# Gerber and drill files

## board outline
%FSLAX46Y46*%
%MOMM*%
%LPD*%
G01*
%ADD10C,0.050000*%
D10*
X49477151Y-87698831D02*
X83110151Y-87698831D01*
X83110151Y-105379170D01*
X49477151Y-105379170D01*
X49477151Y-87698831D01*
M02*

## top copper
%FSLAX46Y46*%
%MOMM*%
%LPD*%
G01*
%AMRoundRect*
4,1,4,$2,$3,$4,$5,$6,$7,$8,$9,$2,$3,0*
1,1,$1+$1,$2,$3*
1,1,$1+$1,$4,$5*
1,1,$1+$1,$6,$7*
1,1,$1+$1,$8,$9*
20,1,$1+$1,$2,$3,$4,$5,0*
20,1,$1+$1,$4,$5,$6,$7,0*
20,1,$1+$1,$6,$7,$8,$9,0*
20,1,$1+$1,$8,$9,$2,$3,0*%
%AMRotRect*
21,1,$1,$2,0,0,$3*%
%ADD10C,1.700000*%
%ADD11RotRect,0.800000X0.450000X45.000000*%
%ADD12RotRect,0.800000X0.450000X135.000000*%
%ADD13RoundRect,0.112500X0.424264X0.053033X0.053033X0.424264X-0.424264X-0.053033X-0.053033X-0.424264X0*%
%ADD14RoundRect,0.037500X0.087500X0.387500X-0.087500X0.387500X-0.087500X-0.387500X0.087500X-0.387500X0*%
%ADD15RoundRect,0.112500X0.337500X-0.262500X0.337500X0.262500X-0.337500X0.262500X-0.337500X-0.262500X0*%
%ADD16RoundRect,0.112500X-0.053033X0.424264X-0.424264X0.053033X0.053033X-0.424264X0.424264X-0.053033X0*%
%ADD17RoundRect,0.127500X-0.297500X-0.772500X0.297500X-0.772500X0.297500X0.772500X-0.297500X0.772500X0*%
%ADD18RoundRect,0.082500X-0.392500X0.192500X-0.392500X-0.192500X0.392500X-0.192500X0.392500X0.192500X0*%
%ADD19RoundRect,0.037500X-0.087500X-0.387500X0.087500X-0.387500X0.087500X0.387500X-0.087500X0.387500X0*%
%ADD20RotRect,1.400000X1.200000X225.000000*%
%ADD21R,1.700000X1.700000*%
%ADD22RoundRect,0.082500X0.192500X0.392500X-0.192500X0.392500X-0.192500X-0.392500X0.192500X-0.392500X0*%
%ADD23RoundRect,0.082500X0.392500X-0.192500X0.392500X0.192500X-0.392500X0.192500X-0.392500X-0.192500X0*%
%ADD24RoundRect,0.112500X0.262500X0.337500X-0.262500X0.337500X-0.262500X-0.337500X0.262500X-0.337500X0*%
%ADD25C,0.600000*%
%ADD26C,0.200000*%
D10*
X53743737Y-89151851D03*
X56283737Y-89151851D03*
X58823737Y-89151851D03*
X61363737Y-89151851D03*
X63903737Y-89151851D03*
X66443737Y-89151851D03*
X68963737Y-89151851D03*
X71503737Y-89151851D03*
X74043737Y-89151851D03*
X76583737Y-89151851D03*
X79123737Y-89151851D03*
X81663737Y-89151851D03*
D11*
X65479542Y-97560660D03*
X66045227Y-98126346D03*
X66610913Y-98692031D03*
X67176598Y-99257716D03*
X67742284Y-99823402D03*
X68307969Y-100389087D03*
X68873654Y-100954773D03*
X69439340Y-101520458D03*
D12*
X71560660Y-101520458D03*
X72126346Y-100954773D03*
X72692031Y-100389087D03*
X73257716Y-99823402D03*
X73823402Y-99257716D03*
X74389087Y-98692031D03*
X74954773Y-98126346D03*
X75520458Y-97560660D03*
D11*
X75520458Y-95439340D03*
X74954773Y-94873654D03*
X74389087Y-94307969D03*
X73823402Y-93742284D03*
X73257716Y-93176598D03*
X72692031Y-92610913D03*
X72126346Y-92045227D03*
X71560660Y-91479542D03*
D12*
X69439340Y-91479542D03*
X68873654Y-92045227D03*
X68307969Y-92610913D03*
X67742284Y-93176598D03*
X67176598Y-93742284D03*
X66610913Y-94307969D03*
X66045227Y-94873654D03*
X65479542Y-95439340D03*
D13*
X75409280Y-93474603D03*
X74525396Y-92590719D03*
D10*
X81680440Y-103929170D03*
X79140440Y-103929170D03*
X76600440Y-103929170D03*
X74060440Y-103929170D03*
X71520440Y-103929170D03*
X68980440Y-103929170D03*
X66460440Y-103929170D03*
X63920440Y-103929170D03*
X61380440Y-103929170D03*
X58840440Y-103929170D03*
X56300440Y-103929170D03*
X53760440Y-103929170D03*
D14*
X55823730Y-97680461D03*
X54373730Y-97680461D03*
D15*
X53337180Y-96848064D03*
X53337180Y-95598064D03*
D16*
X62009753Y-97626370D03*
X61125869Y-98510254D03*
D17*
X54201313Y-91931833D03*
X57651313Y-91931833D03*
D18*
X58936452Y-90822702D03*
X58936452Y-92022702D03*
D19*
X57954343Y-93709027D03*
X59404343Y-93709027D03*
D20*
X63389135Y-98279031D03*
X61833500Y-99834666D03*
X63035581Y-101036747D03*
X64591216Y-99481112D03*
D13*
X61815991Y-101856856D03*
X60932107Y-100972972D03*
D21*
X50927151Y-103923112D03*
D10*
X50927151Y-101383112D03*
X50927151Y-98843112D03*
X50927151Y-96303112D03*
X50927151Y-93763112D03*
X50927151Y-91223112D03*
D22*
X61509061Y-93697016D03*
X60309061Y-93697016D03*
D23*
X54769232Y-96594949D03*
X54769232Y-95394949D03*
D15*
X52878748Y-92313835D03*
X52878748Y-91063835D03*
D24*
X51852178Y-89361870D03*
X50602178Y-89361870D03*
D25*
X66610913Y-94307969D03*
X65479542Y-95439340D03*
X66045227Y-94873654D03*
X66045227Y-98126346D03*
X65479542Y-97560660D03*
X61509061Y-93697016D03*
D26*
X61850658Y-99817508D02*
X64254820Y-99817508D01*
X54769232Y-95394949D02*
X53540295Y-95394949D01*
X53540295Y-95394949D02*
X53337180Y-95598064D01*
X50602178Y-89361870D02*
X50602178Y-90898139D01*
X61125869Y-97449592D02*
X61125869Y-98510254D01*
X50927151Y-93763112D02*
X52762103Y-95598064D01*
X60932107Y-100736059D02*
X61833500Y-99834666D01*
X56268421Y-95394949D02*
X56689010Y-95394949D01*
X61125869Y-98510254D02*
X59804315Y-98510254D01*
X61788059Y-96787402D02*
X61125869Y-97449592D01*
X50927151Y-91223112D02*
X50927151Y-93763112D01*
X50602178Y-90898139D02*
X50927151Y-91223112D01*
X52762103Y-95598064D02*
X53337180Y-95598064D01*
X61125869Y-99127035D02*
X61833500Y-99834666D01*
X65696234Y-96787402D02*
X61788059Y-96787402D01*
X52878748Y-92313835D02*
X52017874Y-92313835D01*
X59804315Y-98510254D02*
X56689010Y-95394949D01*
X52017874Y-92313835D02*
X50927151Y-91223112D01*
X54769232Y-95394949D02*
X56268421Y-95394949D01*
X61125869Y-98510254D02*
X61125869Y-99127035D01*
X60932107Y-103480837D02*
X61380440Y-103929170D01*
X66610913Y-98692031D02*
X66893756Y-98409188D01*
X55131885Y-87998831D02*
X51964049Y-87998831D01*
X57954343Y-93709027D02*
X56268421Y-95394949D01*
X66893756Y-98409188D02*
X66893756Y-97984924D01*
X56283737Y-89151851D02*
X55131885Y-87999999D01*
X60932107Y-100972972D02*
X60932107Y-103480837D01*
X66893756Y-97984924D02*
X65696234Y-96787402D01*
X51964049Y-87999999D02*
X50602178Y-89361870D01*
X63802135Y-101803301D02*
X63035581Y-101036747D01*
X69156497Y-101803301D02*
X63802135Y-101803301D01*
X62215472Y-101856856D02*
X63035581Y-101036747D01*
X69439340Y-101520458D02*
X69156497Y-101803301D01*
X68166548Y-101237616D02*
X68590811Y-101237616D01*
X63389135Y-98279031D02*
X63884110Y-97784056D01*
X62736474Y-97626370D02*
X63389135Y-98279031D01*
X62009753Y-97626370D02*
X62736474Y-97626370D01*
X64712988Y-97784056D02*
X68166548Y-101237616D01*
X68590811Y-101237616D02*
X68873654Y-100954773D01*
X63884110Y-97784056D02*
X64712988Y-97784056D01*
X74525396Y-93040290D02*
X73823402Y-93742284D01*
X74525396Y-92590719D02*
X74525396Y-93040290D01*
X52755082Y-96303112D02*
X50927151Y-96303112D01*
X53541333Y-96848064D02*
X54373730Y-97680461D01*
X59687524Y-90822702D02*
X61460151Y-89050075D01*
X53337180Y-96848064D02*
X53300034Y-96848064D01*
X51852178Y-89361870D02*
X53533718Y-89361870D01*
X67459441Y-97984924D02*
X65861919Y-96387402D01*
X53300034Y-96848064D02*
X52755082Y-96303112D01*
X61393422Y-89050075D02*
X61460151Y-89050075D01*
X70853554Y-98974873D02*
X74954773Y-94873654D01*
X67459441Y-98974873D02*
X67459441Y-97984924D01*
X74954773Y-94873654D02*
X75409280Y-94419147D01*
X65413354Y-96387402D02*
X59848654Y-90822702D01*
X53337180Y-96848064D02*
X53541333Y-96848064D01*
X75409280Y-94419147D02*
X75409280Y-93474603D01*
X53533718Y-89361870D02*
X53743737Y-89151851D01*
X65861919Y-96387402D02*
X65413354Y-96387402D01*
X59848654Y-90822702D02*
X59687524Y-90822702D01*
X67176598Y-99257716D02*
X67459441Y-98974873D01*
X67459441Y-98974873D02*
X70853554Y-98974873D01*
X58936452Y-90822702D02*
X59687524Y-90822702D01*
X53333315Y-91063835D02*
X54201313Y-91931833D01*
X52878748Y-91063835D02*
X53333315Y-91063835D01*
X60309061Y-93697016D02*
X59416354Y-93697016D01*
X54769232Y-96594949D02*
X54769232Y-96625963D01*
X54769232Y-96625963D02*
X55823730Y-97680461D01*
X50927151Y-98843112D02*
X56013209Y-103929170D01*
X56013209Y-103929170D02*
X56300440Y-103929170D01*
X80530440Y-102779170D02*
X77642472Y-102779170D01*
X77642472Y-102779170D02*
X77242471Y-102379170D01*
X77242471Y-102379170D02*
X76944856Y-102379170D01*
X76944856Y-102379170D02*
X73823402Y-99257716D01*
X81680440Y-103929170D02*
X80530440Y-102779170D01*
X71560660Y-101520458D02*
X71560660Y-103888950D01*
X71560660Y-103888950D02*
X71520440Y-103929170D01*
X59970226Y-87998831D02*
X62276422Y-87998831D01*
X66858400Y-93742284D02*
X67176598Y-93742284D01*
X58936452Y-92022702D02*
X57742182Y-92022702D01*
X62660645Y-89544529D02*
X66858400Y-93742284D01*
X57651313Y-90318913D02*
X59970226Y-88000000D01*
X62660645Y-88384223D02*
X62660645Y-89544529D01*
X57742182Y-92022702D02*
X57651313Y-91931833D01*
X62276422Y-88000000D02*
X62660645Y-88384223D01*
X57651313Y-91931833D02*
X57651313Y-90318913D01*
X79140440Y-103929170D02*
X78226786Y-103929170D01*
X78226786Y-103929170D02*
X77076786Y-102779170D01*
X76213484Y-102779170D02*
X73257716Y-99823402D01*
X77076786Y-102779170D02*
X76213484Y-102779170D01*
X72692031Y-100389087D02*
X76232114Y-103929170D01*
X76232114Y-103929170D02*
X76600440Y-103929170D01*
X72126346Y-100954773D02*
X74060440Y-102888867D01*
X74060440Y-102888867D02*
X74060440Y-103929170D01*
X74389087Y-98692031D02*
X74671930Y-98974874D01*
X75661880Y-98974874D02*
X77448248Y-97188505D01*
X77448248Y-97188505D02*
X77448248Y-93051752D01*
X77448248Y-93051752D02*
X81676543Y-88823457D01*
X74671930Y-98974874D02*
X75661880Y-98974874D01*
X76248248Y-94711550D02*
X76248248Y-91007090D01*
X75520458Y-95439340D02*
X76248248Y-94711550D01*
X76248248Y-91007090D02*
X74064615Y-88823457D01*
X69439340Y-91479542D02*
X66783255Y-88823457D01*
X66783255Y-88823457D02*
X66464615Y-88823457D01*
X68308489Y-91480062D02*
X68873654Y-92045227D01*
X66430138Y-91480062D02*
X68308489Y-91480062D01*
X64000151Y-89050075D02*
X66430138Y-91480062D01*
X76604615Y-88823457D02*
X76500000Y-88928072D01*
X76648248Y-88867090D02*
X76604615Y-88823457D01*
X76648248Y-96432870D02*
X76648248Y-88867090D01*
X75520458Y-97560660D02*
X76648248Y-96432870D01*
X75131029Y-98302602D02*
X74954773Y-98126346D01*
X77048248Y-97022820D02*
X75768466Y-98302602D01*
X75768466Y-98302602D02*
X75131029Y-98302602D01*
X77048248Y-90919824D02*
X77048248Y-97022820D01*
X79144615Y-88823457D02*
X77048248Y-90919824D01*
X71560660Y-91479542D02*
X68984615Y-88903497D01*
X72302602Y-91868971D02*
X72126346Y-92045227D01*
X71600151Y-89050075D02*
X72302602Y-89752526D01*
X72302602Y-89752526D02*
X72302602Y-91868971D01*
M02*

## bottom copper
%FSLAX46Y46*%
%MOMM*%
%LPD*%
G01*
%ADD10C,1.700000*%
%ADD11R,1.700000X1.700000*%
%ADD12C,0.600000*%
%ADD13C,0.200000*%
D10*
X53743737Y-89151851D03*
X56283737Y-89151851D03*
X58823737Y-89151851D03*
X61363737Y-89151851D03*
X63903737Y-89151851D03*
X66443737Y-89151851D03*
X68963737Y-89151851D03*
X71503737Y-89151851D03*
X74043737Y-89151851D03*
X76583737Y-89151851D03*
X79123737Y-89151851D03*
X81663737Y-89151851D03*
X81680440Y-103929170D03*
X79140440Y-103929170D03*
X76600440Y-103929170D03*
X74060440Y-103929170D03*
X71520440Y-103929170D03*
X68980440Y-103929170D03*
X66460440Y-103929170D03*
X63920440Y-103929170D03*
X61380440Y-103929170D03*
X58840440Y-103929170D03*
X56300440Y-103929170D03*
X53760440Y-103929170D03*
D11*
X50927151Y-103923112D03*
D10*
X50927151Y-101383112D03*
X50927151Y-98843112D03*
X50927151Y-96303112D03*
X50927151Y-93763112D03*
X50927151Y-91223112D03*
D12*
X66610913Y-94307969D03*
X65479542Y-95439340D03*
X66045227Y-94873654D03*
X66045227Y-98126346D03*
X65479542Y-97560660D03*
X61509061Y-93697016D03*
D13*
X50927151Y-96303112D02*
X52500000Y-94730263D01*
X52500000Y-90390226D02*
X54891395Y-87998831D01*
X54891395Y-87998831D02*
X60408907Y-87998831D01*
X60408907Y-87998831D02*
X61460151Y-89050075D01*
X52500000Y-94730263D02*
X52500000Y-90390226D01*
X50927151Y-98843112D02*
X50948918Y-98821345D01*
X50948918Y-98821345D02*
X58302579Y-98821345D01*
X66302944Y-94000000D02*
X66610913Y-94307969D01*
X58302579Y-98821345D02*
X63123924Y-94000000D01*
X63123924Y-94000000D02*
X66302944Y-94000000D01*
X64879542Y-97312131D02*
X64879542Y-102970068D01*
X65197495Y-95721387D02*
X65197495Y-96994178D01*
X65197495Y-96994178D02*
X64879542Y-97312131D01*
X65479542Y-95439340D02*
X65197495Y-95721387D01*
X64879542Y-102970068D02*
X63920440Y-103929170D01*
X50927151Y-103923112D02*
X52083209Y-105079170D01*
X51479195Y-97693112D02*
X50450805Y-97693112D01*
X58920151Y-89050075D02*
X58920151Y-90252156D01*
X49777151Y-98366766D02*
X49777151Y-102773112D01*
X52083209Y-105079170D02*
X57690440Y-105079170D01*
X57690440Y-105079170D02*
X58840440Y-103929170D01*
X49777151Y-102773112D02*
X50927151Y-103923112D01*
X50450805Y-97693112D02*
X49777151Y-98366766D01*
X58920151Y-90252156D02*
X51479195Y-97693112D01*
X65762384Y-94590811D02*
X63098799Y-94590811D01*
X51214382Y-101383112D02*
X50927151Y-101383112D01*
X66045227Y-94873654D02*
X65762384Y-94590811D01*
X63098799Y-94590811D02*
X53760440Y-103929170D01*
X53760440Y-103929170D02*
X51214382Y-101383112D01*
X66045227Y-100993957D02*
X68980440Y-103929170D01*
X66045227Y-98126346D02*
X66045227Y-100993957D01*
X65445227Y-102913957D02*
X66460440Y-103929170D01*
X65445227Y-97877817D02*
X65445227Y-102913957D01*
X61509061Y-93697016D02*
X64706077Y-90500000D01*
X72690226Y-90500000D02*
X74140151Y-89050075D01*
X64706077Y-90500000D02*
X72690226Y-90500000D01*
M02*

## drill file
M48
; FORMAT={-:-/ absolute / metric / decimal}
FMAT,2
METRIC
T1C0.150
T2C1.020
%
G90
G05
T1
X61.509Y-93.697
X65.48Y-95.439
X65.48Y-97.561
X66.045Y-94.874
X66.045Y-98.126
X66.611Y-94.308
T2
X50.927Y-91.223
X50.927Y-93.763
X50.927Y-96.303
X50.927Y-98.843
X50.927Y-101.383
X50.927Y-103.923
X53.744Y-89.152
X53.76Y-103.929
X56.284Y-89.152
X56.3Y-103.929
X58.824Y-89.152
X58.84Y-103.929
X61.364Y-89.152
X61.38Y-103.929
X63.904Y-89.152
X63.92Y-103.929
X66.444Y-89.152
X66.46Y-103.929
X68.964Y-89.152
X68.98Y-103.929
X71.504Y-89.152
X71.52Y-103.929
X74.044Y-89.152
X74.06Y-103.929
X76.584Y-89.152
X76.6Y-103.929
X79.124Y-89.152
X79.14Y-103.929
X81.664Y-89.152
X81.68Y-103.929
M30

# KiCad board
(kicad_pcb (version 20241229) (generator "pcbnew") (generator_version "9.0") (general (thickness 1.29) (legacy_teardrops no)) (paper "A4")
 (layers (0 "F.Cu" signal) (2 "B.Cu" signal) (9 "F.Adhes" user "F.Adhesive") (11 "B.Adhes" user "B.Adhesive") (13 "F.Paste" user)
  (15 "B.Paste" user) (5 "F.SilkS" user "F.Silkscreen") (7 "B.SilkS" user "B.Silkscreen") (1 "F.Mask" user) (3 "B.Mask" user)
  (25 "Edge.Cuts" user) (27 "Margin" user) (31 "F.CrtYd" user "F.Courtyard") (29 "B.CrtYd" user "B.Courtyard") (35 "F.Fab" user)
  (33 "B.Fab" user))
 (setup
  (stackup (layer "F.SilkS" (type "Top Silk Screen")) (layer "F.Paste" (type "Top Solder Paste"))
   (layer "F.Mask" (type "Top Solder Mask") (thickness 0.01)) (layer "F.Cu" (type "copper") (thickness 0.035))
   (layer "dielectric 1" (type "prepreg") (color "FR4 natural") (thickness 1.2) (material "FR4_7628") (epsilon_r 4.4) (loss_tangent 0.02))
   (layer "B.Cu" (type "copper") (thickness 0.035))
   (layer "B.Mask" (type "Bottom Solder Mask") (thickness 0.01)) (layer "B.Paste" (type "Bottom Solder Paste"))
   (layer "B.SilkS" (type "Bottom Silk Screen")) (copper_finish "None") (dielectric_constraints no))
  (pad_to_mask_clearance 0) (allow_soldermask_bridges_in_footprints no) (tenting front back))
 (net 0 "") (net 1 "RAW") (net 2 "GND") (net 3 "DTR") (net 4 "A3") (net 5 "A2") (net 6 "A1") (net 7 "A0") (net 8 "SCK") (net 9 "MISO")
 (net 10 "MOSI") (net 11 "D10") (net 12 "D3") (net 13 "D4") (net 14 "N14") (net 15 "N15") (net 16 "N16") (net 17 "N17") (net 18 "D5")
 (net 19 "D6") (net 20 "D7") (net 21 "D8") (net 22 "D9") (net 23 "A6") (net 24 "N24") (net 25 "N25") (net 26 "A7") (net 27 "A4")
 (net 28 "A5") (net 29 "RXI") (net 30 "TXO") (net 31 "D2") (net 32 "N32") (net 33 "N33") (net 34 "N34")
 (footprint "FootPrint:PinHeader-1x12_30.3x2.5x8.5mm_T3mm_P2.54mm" (layer "F.Cu") (at 67.703737 89.151851)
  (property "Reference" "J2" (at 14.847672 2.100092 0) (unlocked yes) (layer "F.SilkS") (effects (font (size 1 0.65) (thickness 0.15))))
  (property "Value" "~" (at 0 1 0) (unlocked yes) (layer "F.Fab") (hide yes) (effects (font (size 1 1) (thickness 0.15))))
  (pad "1" thru_hole circle (at -13.96 0) (size 1.7 1.7) (drill 1.02) (layers "*.Cu" "*.Mask") (remove_unused_layers no) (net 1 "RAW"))
  (pad "2" thru_hole circle (at -11.42 0) (size 1.7 1.7) (drill 1.02) (layers "*.Cu" "*.Mask") (remove_unused_layers no) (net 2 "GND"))
  (pad "3" thru_hole circle (at -8.88 0) (size 1.7 1.7) (drill 1.02) (layers "*.Cu" "*.Mask") (remove_unused_layers no) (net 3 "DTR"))
  (pad "4" thru_hole circle (at -6.34 0) (size 1.7 1.7) (drill 1.02) (layers "*.Cu" "*.Mask") (remove_unused_layers no) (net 1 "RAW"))
  (pad "5" thru_hole circle (at -3.8 0) (size 1.7 1.7) (drill 1.02) (layers "*.Cu" "*.Mask") (remove_unused_layers no) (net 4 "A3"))
  (pad "6" thru_hole circle (at -1.26 0) (size 1.7 1.7) (drill 1.02) (layers "*.Cu" "*.Mask") (remove_unused_layers no) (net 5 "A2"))
  (pad "7" thru_hole circle (at 1.26 0) (size 1.7 1.7) (drill 1.02) (layers "*.Cu" "*.Mask") (remove_unused_layers no) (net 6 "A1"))
  (pad "8" thru_hole circle (at 3.8 0) (size 1.7 1.7) (drill 1.02) (layers "*.Cu" "*.Mask") (remove_unused_layers no) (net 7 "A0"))
  (pad "9" thru_hole circle (at 6.34 0) (size 1.7 1.7) (drill 1.02) (layers "*.Cu" "*.Mask") (remove_unused_layers no) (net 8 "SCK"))
  (pad "10" thru_hole circle (at 8.88 0) (size 1.7 1.7) (drill 1.02) (layers "*.Cu" "*.Mask") (remove_unused_layers no) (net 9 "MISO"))
  (pad "11" thru_hole circle (at 11.42 0) (size 1.7 1.7) (drill 1.02) (layers "*.Cu" "*.Mask") (remove_unused_layers no) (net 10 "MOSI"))
  (pad "12" thru_hole circle (at 13.96 0) (size 1.7 1.7) (drill 1.02) (layers "*.Cu" "*.Mask") (remove_unused_layers no) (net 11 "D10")))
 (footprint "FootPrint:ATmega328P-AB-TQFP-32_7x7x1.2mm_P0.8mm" (layer "F.Cu") (at 70.5 96.5 45)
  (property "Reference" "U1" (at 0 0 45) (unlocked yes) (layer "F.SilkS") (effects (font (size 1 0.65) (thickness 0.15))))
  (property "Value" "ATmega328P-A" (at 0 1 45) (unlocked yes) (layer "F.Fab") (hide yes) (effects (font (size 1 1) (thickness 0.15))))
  (pad "1" smd rect (at -4.3 -2.8 45) (size 0.8 0.45) (layers "F.Cu" "F.Mask" "F.Paste") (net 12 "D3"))
  (pad "2" smd rect (at -4.3 -2 45) (size 0.8 0.45) (layers "F.Cu" "F.Mask" "F.Paste") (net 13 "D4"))
  (pad "3" smd rect (at -4.3 -1.2 45) (size 0.8 0.45) (layers "F.Cu" "F.Mask" "F.Paste") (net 2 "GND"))
  (pad "4" smd rect (at -4.3 -0.4 45) (size 0.8 0.45) (layers "F.Cu" "F.Mask" "F.Paste") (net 1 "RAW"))
  (pad "5" smd rect (at -4.3 0.4 45) (size 0.8 0.45) (layers "F.Cu" "F.Mask" "F.Paste") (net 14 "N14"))
  (pad "6" smd rect (at -4.3 1.2 45) (size 0.8 0.45) (layers "F.Cu" "F.Mask" "F.Paste") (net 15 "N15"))
  (pad "7" smd rect (at -4.3 2 45) (size 0.8 0.45) (layers "F.Cu" "F.Mask" "F.Paste") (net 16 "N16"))
  (pad "8" smd rect (at -4.3 2.8 45) (size 0.8 0.45) (layers "F.Cu" "F.Mask" "F.Paste") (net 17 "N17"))
  (pad "9" smd rect (at -2.8 4.3 135) (size 0.8 0.45) (layers "F.Cu" "F.Mask" "F.Paste") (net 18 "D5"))
  (pad "10" smd rect (at -2 4.3 135) (size 0.8 0.45) (layers "F.Cu" "F.Mask" "F.Paste") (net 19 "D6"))
  (pad "11" smd rect (at -1.2 4.3 135) (size 0.8 0.45) (layers "F.Cu" "F.Mask" "F.Paste") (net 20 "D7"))
  (pad "12" smd rect (at -0.4 4.3 135) (size 0.8 0.45) (layers "F.Cu" "F.Mask" "F.Paste") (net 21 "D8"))
  (pad "13" smd rect (at 0.4 4.3 135) (size 0.8 0.45) (layers "F.Cu" "F.Mask" "F.Paste") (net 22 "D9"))
  (pad "14" smd rect (at 1.2 4.3 135) (size 0.8 0.45) (layers "F.Cu" "F.Mask" "F.Paste") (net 11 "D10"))
  (pad "15" smd rect (at 2 4.3 135) (size 0.8 0.45) (layers "F.Cu" "F.Mask" "F.Paste") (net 10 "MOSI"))
  (pad "16" smd rect (at 2.8 4.3 135) (size 0.8 0.45) (layers "F.Cu" "F.Mask" "F.Paste") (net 9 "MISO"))
  (pad "17" smd rect (at 4.3 2.8 45) (size 0.8 0.45) (layers "F.Cu" "F.Mask" "F.Paste") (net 8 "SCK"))
  (pad "18" smd rect (at 4.3 2 45) (size 0.8 0.45) (layers "F.Cu" "F.Mask" "F.Paste") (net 1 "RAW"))
  (pad "19" smd rect (at 4.3 1.2 45) (size 0.8 0.45) (layers "F.Cu" "F.Mask" "F.Paste") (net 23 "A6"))
  (pad "20" smd rect (at 4.3 0.4 45) (size 0.8 0.45) (layers "F.Cu" "F.Mask" "F.Paste") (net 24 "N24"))
  (pad "21" smd rect (at 4.3 -0.4 45) (size 0.8 0.45) (layers "F.Cu" "F.Mask" "F.Paste") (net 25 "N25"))
  (pad "22" smd rect (at 4.3 -1.2 45) (size 0.8 0.45) (layers "F.Cu" "F.Mask" "F.Paste") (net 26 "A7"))
  (pad "23" smd rect (at 4.3 -2 45) (size 0.8 0.45) (layers "F.Cu" "F.Mask" "F.Paste") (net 7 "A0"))
  (pad "24" smd rect (at 4.3 -2.8 45) (size 0.8 0.45) (layers "F.Cu" "F.Mask" "F.Paste") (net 6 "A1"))
  (pad "25" smd rect (at 2.8 -4.3 135) (size 0.8 0.45) (layers "F.Cu" "F.Mask" "F.Paste") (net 5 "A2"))
  (pad "26" smd rect (at 2 -4.3 135) (size 0.8 0.45) (layers "F.Cu" "F.Mask" "F.Paste") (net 4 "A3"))
  (pad "27" smd rect (at 1.2 -4.3 135) (size 0.8 0.45) (layers "F.Cu" "F.Mask" "F.Paste") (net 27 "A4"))
  (pad "28" smd rect (at 0.4 -4.3 135) (size 0.8 0.45) (layers "F.Cu" "F.Mask" "F.Paste") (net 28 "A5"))
  (pad "29" smd rect (at -0.4 -4.3 135) (size 0.8 0.45) (layers "F.Cu" "F.Mask" "F.Paste") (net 3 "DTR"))
  (pad "30" smd rect (at -1.2 -4.3 135) (size 0.8 0.45) (layers "F.Cu" "F.Mask" "F.Paste") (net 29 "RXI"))
  (pad "31" smd rect (at -2 -4.3 135) (size 0.8 0.45) (layers "F.Cu" "F.Mask" "F.Paste") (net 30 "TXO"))
  (pad "32" smd rect (at -2.8 -4.3 135) (size 0.8 0.45) (layers "F.Cu" "F.Mask" "F.Paste") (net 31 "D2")))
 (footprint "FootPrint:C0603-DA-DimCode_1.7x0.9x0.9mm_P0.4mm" (layer "F.Cu") (at 74.967338 93.032661 135)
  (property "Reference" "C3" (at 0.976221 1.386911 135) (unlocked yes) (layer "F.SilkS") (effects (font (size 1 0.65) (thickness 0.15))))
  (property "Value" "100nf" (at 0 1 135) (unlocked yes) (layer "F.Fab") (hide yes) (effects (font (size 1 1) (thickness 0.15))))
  (pad "1" smd roundrect (at -0.625 0 135) (size 0.75 0.9) (layers "F.Cu" "F.Mask" "F.Paste") (roundrect_rratio 0.15) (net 1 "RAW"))
  (pad "2" smd roundrect (at 0.625 0 135) (size 0.75 0.9) (layers "F.Cu" "F.Mask" "F.Paste") (roundrect_rratio 0.15) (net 24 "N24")))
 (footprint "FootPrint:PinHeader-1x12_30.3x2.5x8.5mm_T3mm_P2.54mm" (layer "F.Cu") (at 67.72044 103.92917 180)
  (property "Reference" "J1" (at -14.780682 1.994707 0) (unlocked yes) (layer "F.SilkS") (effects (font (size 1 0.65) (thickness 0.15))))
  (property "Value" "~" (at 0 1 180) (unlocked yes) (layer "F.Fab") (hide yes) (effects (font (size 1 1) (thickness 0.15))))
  (pad "1" thru_hole circle (at -13.96 0 180) (size 1.7 1.7) (drill 1.02) (layers "*.Cu" "*.Mask") (remove_unused_layers no) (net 22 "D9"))
  (pad "2" thru_hole circle (at -11.42 0 180) (size 1.7 1.7) (drill 1.02) (layers "*.Cu" "*.Mask") (remove_unused_layers no) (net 21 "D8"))
  (pad "3" thru_hole circle (at -8.88 0 180) (size 1.7 1.7) (drill 1.02) (layers "*.Cu" "*.Mask") (remove_unused_layers no) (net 20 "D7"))
  (pad "4" thru_hole circle (at -6.34 0 180) (size 1.7 1.7) (drill 1.02) (layers "*.Cu" "*.Mask") (remove_unused_layers no) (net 19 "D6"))
  (pad "5" thru_hole circle (at -3.8 0 180) (size 1.7 1.7) (drill 1.02) (layers "*.Cu" "*.Mask") (remove_unused_layers no) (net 18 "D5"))
  (pad "6" thru_hole circle (at -1.26 0 180) (size 1.7 1.7) (drill 1.02) (layers "*.Cu" "*.Mask") (remove_unused_layers no) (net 13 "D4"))
  (pad "7" thru_hole circle (at 1.26 0 180) (size 1.7 1.7) (drill 1.02) (layers "*.Cu" "*.Mask") (remove_unused_layers no) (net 12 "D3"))
  (pad "8" thru_hole circle (at 3.8 0 180) (size 1.7 1.7) (drill 1.02) (layers "*.Cu" "*.Mask") (remove_unused_layers no) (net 31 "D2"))
  (pad "9" thru_hole circle (at 6.34 0 180) (size 1.7 1.7) (drill 1.02) (layers "*.Cu" "*.Mask") (remove_unused_layers no) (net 2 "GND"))
  (pad "10" thru_hole circle (at 8.88 0 180) (size 1.7 1.7) (drill 1.02) (layers "*.Cu" "*.Mask") (remove_unused_layers no) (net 3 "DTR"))
  (pad "11" thru_hole circle (at 11.42 0 180) (size 1.7 1.7) (drill 1.02) (layers "*.Cu" "*.Mask") (remove_unused_layers no) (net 29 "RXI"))
  (pad "12" thru_hole circle (at 13.96 0 180) (size 1.7 1.7) (drill 1.02) (layers "*.Cu" "*.Mask") (remove_unused_layers no) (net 30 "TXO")))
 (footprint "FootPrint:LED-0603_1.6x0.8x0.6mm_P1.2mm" (layer "F.Cu") (at 55.09873 97.680461 180)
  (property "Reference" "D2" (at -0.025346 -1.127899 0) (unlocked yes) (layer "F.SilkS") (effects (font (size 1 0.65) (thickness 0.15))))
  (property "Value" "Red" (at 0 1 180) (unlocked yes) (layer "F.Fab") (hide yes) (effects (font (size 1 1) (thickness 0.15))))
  (pad "1" smd roundrect (at -0.725 0 180) (size 0.25 0.85) (layers "F.Cu" "F.Mask" "F.Paste") (roundrect_rratio 0.15) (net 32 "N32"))
  (pad "2" smd roundrect (at 0.725 0 180) (size 0.25 0.85) (layers "F.Cu" "F.Mask" "F.Paste") (roundrect_rratio 0.15) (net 1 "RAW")))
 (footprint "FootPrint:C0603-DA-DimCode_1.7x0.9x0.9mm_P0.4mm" (layer "F.Cu") (at 53.33718 96.223064 90)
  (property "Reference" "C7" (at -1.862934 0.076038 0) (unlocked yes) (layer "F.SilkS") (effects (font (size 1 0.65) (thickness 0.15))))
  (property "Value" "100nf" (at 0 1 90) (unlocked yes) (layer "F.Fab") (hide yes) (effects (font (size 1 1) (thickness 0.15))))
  (pad "1" smd roundrect (at -0.625 0 90) (size 0.75 0.9) (layers "F.Cu" "F.Mask" "F.Paste") (roundrect_rratio 0.15) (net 1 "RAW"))
  (pad "2" smd roundrect (at 0.625 0 90) (size 0.75 0.9) (layers "F.Cu" "F.Mask" "F.Paste") (roundrect_rratio 0.15) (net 2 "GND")))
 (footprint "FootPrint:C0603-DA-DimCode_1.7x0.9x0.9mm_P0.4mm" (layer "F.Cu") (at 61.567811 98.068312 -135)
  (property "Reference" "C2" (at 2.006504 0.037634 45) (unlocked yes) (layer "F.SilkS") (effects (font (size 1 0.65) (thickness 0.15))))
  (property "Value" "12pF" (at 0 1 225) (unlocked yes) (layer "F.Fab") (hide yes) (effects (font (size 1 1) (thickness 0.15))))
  (pad "1" smd roundrect (at -0.625 0 225) (size 0.75 0.9) (layers "F.Cu" "F.Mask" "F.Paste") (roundrect_rratio 0.15) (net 16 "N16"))
  (pad "2" smd roundrect (at 0.625 0 225) (size 0.75 0.9) (layers "F.Cu" "F.Mask" "F.Paste") (roundrect_rratio 0.15) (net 2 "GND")))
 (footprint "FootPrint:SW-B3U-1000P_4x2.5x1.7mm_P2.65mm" (layer "F.Cu") (at 55.926313 91.931833)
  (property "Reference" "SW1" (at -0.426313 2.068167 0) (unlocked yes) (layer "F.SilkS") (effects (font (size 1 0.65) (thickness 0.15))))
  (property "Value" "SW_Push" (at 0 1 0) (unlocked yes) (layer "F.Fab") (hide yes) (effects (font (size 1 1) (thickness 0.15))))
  (pad "1" smd roundrect (at -1.725 0) (size 0.85 1.8) (layers "F.Cu" "F.Mask" "F.Paste") (roundrect_rratio 0.15) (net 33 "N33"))
  (pad "2" smd roundrect (at 1.725 0) (size 0.85 1.8) (layers "F.Cu" "F.Mask" "F.Paste") (roundrect_rratio 0.15) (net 3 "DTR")))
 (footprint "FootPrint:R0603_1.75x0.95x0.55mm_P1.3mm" (layer "F.Cu") (at 58.936452 91.422702 -90)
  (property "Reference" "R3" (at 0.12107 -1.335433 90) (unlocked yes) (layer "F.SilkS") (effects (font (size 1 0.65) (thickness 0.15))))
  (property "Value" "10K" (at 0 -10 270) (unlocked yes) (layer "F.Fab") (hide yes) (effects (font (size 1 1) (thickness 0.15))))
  (pad "1" smd roundrect (at -0.6 0 270) (size 0.55 0.95) (layers "F.Cu" "F.Mask" "F.Paste") (roundrect_rratio 0.15) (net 1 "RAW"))
  (pad "2" smd roundrect (at 0.6 0 270) (size 0.55 0.95) (layers "F.Cu" "F.Mask" "F.Paste") (roundrect_rratio 0.15) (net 3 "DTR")))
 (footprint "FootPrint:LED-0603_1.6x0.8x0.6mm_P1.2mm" (layer "F.Cu") (at 58.679343 93.709027)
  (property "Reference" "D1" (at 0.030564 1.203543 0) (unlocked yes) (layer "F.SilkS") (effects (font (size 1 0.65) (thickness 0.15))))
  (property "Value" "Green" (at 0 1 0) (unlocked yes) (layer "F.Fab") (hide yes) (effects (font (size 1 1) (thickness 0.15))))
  (pad "1" smd roundrect (at -0.725 0) (size 0.25 0.85) (layers "F.Cu" "F.Mask" "F.Paste") (roundrect_rratio 0.15) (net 2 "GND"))
  (pad "2" smd roundrect (at 0.725 0) (size 0.25 0.85) (layers "F.Cu" "F.Mask" "F.Paste") (roundrect_rratio 0.15) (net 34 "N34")))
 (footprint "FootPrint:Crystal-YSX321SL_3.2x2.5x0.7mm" (layer "F.Cu") (at 63.212358 99.657889 -135)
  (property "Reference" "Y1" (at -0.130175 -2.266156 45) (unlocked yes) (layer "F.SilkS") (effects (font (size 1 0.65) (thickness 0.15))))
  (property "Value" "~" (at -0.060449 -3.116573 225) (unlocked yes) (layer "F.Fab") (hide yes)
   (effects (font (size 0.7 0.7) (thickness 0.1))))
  (pad "1" smd rect (at -1.1 0.85 225) (size 1.4 1.2) (layers "F.Cu" "F.Mask" "F.Paste") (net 16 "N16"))
  (pad "2" smd rect (at 1.1 0.85 225) (size 1.4 1.2) (layers "F.Cu" "F.Mask" "F.Paste") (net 2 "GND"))
  (pad "3" smd rect (at 1.1 -0.85 225) (size 1.4 1.2) (layers "F.Cu" "F.Mask" "F.Paste") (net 17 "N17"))
  (pad "4" smd rect (at -1.1 -0.85 225) (size 1.4 1.2) (layers "F.Cu" "F.Mask" "F.Paste") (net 2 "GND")))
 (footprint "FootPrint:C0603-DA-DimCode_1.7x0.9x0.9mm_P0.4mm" (layer "F.Cu") (at 61.374049 101.414914 135)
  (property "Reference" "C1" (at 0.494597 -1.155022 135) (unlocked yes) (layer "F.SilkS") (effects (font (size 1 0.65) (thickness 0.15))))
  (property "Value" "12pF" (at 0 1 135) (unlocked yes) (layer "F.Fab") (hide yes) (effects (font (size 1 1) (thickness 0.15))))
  (pad "1" smd roundrect (at -0.625 0 135) (size 0.75 0.9) (layers "F.Cu" "F.Mask" "F.Paste") (roundrect_rratio 0.15) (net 17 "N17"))
  (pad "2" smd roundrect (at 0.625 0 135) (size 0.75 0.9) (layers "F.Cu" "F.Mask" "F.Paste") (roundrect_rratio 0.15) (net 2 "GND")))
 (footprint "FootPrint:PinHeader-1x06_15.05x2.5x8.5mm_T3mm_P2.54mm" (layer "F.Cu") (at 50.927151 97.573112 90)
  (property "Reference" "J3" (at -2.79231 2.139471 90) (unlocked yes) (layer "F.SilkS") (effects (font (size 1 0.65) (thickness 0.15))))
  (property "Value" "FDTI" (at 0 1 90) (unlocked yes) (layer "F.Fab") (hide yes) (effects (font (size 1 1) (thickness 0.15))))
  (pad "1" thru_hole rect (at -6.35 0 90) (size 1.7 1.7) (drill 1.02) (layers "*.Cu" "*.Mask") (remove_unused_layers no) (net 3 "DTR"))
  (pad "2" thru_hole circle (at -3.81 0 90) (size 1.7 1.7) (drill 1.02) (layers "*.Cu" "*.Mask") (remove_unused_layers no) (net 30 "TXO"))
  (pad "3" thru_hole circle (at -1.27 0 90) (size 1.7 1.7) (drill 1.02) (layers "*.Cu" "*.Mask") (remove_unused_layers no) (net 29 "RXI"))
  (pad "4" thru_hole circle (at 1.27 0 90) (size 1.7 1.7) (drill 1.02) (layers "*.Cu" "*.Mask") (remove_unused_layers no) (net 1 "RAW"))
  (pad "5" thru_hole circle (at 3.81 0 90) (size 1.7 1.7) (drill 1.02) (layers "*.Cu" "*.Mask") (remove_unused_layers no) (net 2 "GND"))
  (pad "6" thru_hole circle (at 6.35 0 90) (size 1.7 1.7) (drill 1.02) (layers "*.Cu" "*.Mask") (remove_unused_layers no) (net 2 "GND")))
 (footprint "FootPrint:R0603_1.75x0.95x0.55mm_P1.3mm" (layer "F.Cu") (at 60.909061 93.697016 180)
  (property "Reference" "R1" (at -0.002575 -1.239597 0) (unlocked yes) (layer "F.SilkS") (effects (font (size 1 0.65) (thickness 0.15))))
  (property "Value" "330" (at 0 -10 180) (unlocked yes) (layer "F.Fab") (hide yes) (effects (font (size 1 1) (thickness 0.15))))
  (pad "1" smd roundrect (at -0.6 0 180) (size 0.55 0.95) (layers "F.Cu" "F.Mask" "F.Paste") (roundrect_rratio 0.15) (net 8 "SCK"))
  (pad "2" smd roundrect (at 0.6 0 180) (size 0.55 0.95) (layers "F.Cu" "F.Mask" "F.Paste") (roundrect_rratio 0.15) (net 34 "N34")))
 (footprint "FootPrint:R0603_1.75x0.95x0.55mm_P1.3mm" (layer "F.Cu") (at 54.769232 95.994949 90)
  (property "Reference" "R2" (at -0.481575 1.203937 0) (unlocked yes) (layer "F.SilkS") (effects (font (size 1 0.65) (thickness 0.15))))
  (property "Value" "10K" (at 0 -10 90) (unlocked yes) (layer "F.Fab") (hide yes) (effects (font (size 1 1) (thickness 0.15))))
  (pad "1" smd roundrect (at -0.6 0 90) (size 0.55 0.95) (layers "F.Cu" "F.Mask" "F.Paste") (roundrect_rratio 0.15) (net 32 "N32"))
  (pad "2" smd roundrect (at 0.6 0 90) (size 0.55 0.95) (layers "F.Cu" "F.Mask" "F.Paste") (roundrect_rratio 0.15) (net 2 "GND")))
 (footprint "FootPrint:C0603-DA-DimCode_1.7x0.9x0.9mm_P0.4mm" (layer "F.Cu") (at 52.878748 91.688835 90)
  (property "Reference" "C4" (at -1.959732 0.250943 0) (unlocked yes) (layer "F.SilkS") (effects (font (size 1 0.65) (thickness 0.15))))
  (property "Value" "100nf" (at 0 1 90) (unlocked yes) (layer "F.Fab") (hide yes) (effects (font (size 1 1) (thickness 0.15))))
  (pad "1" smd roundrect (at -0.625 0 90) (size 0.75 0.9) (layers "F.Cu" "F.Mask" "F.Paste") (roundrect_rratio 0.15) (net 2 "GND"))
  (pad "2" smd roundrect (at 0.625 0 90) (size 0.75 0.9) (layers "F.Cu" "F.Mask" "F.Paste") (roundrect_rratio 0.15) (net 33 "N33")))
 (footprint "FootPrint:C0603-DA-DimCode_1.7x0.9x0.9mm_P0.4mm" (layer "F.Cu") (at 51.227178 89.36187 180)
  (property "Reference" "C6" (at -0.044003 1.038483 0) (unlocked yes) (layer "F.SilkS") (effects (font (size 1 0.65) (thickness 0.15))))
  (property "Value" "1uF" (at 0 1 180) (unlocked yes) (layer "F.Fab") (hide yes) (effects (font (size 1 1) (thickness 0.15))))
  (pad "1" smd roundrect (at -0.625 0 180) (size 0.75 0.9) (layers "F.Cu" "F.Mask" "F.Paste") (roundrect_rratio 0.15) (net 1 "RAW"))
  (pad "2" smd roundrect (at 0.625 0 180) (size 0.75 0.9) (layers "F.Cu" "F.Mask" "F.Paste") (roundrect_rratio 0.15) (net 2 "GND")))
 (gr_rect (start 49.477151 87.698831) (end 83.110151 105.37917) (stroke (width 0.05) (type solid)) (fill no) (layer "Edge.Cuts"))
 (segment (start 61.850658 99.817508) (end 64.25482 99.817508) (width 0.2) (layer "F.Cu") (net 2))
 (segment (start 54.769232 95.394949) (end 53.540295 95.394949) (width 0.2) (layer "F.Cu") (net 2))
 (segment (start 53.540295 95.394949) (end 53.33718 95.598064) (width 0.2) (layer "F.Cu") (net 2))
 (segment (start 50.602178 89.36187) (end 50.602178 90.898139) (width 0.2) (layer "F.Cu") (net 2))
 (segment (start 61.125869 97.449592) (end 61.125869 98.510254) (width 0.2) (layer "F.Cu") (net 2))
 (segment (start 50.927151 93.763112) (end 52.762103 95.598064) (width 0.2) (layer "F.Cu") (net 2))
 (segment (start 60.932107 100.736059) (end 61.8335 99.834666) (width 0.2) (layer "F.Cu") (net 2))
 (segment (start 56.268421 95.394949) (end 56.68901 95.394949) (width 0.2) (layer "F.Cu") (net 2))
 (segment (start 61.125869 98.510254) (end 59.804315 98.510254) (width 0.2) (layer "F.Cu") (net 2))
 (segment (start 61.788059 96.787402) (end 61.125869 97.449592) (width 0.2) (layer "F.Cu") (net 2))
 (segment (start 50.927151 91.223112) (end 50.927151 93.763112) (width 0.2) (layer "F.Cu") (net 2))
 (segment (start 50.602178 90.898139) (end 50.927151 91.223112) (width 0.2) (layer "F.Cu") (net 2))
 (segment (start 52.762103 95.598064) (end 53.33718 95.598064) (width 0.2) (layer "F.Cu") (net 2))
 (segment (start 61.125869 99.127035) (end 61.8335 99.834666) (width 0.2) (layer "F.Cu") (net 2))
 (segment (start 65.696234 96.787402) (end 61.788059 96.787402) (width 0.2) (layer "F.Cu") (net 2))
 (segment (start 52.878748 92.313835) (end 52.017874 92.313835) (width 0.2) (layer "F.Cu") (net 2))
 (segment (start 59.804315 98.510254) (end 56.68901 95.394949) (width 0.2) (layer "F.Cu") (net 2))
 (segment (start 52.017874 92.313835) (end 50.927151 91.223112) (width 0.2) (layer "F.Cu") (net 2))
 (segment (start 54.769232 95.394949) (end 56.268421 95.394949) (width 0.2) (layer "F.Cu") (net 2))
 (segment (start 61.125869 98.510254) (end 61.125869 99.127035) (width 0.2) (layer "F.Cu") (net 2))
 (segment (start 60.932107 103.480837) (end 61.38044 103.92917) (width 0.2) (layer "F.Cu") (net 2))
 (segment (start 66.610913 98.692031) (end 66.893756 98.409188) (width 0.2) (layer "F.Cu") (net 2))
 (segment (start 55.131885 87.998831) (end 51.964049 87.998831) (width 0.2) (layer "F.Cu") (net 2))
 (segment (start 57.954343 93.709027) (end 56.268421 95.394949) (width 0.2) (layer "F.Cu") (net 2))
 (segment (start 66.893756 98.409188) (end 66.893756 97.984924) (width 0.2) (layer "F.Cu") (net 2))
 (segment (start 56.283737 89.151851) (end 55.131885 87.999999) (width 0.2) (layer "F.Cu") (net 2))
 (segment (start 60.932107 100.972972) (end 60.932107 103.480837) (width 0.2) (layer "F.Cu") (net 2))
 (segment (start 66.893756 97.984924) (end 65.696234 96.787402) (width 0.2) (layer "F.Cu") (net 2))
 (segment (start 51.964049 87.999999) (end 50.602178 89.36187) (width 0.2) (layer "F.Cu") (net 2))
 (segment (start 63.802135 101.803301) (end 63.035581 101.036747) (width 0.2) (layer "F.Cu") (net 17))
 (segment (start 69.156497 101.803301) (end 63.802135 101.803301) (width 0.2) (layer "F.Cu") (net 17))
 (segment (start 62.215472 101.856856) (end 63.035581 101.036747) (width 0.2) (layer "F.Cu") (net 17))
 (segment (start 69.43934 101.520458) (end 69.156497 101.803301) (width 0.2) (layer "F.Cu") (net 17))
 (segment (start 68.166548 101.237616) (end 68.590811 101.237616) (width 0.2) (layer "F.Cu") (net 16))
 (segment (start 63.389135 98.279031) (end 63.88411 97.784056) (width 0.2) (layer "F.Cu") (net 16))
 (segment (start 62.736474 97.62637) (end 63.389135 98.279031) (width 0.2) (layer "F.Cu") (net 16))
 (segment (start 62.009753 97.62637) (end 62.736474 97.62637) (width 0.2) (layer "F.Cu") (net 16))
 (segment (start 64.712988 97.784056) (end 68.166548 101.237616) (width 0.2) (layer "F.Cu") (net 16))
 (segment (start 68.590811 101.237616) (end 68.873654 100.954773) (width 0.2) (layer "F.Cu") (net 16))
 (segment (start 63.88411 97.784056) (end 64.712988 97.784056) (width 0.2) (layer "F.Cu") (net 16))
 (segment (start 74.525396 93.04029) (end 73.823402 93.742284) (width 0.2) (layer "F.Cu") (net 24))
 (segment (start 74.525396 92.590719) (end 74.525396 93.04029) (width 0.2) (layer "F.Cu") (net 24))
 (segment (start 52.755082 96.303112) (end 50.927151 96.303112) (width 0.2) (layer "F.Cu") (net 1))
 (segment (start 53.541333 96.848064) (end 54.37373 97.680461) (width 0.2) (layer "F.Cu") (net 1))
 (segment (start 59.687524 90.822702) (end 61.460151 89.050075) (width 0.2) (layer "F.Cu") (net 1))
 (segment (start 53.33718 96.848064) (end 53.300034 96.848064) (width 0.2) (layer "F.Cu") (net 1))
 (segment (start 51.852178 89.36187) (end 53.533718 89.36187) (width 0.2) (layer "F.Cu") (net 1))
 (segment (start 67.459441 97.984924) (end 65.861919 96.387402) (width 0.2) (layer "F.Cu") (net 1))
 (segment (start 53.300034 96.848064) (end 52.755082 96.303112) (width 0.2) (layer "F.Cu") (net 1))
 (segment (start 61.393422 89.050075) (end 61.460151 89.050075) (width 0.2) (layer "F.Cu") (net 1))
 (segment (start 70.853554 98.974873) (end 74.954773 94.873654) (width 0.2) (layer "F.Cu") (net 1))
 (segment (start 67.459441 98.974873) (end 67.459441 97.984924) (width 0.2) (layer "F.Cu") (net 1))
 (segment (start 74.954773 94.873654) (end 75.40928 94.419147) (width 0.2) (layer "F.Cu") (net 1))
 (segment (start 65.413354 96.387402) (end 59.848654 90.822702) (width 0.2) (layer "F.Cu") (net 1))
 (segment (start 53.33718 96.848064) (end 53.541333 96.848064) (width 0.2) (layer "F.Cu") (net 1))
 (segment (start 75.40928 94.419147) (end 75.40928 93.474603) (width 0.2) (layer "F.Cu") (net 1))
 (segment (start 53.533718 89.36187) (end 53.743737 89.151851) (width 0.2) (layer "F.Cu") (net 1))
 (segment (start 65.861919 96.387402) (end 65.413354 96.387402) (width 0.2) (layer "F.Cu") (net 1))
 (segment (start 59.848654 90.822702) (end 59.687524 90.822702) (width 0.2) (layer "F.Cu") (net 1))
 (segment (start 67.176598 99.257716) (end 67.459441 98.974873) (width 0.2) (layer "F.Cu") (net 1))
 (segment (start 67.459441 98.974873) (end 70.853554 98.974873) (width 0.2) (layer "F.Cu") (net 1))
 (segment (start 58.936452 90.822702) (end 59.687524 90.822702) (width 0.2) (layer "F.Cu") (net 1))
 (segment (start 50.927151 96.303112) (end 52.5 94.730263) (width 0.2) (layer "B.Cu") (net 1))
 (segment (start 52.5 90.390226) (end 54.891395 87.998831) (width 0.2) (layer "B.Cu") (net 1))
 (segment (start 54.891395 87.998831) (end 60.408907 87.998831) (width 0.2) (layer "B.Cu") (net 1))
 (segment (start 60.408907 87.998831) (end 61.460151 89.050075) (width 0.2) (layer "B.Cu") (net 1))
 (segment (start 52.5 94.730263) (end 52.5 90.390226) (width 0.2) (layer "B.Cu") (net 1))
 (segment (start 53.333315 91.063835) (end 54.201313 91.931833) (width 0.2) (layer "F.Cu") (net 33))
 (segment (start 52.878748 91.063835) (end 53.333315 91.063835) (width 0.2) (layer "F.Cu") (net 33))
 (segment (start 60.309061 93.697016) (end 59.416354 93.697016) (width 0.2) (layer "F.Cu") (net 34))
 (segment (start 54.769232 96.594949) (end 54.769232 96.625963) (width 0.2) (layer "F.Cu") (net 32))
 (segment (start 54.769232 96.625963) (end 55.82373 97.680461) (width 0.2) (layer "F.Cu") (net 32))
 (segment (start 50.927151 98.843112) (end 56.013209 103.92917) (width 0.2) (layer "F.Cu") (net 29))
 (segment (start 56.013209 103.92917) (end 56.30044 103.92917) (width 0.2) (layer "F.Cu") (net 29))
 (via (at 66.610913 94.307969) (size 0.6) (drill 0.15) (layers "F.Cu" "B.Cu") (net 29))
 (segment (start 50.927151 98.843112) (end 50.948918 98.821345) (width 0.2) (layer "B.Cu") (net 29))
 (segment (start 50.948918 98.821345) (end 58.302579 98.821345) (width 0.2) (layer "B.Cu") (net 29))
 (segment (start 66.302944 94) (end 66.610913 94.307969) (width 0.2) (layer "B.Cu") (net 29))
 (segment (start 58.302579 98.821345) (end 63.123924 94) (width 0.2) (layer "B.Cu") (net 29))
 (segment (start 63.123924 94) (end 66.302944 94) (width 0.2) (layer "B.Cu") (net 29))
 (segment (start 80.53044 102.77917) (end 77.642472 102.77917) (width 0.2) (layer "F.Cu") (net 22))
 (segment (start 77.642472 102.77917) (end 77.242471 102.37917) (width 0.2) (layer "F.Cu") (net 22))
 (segment (start 77.242471 102.37917) (end 76.944856 102.37917) (width 0.2) (layer "F.Cu") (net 22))
 (segment (start 76.944856 102.37917) (end 73.823402 99.257716) (width 0.2) (layer "F.Cu") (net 22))
 (segment (start 81.68044 103.92917) (end 80.53044 102.77917) (width 0.2) (layer "F.Cu") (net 22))
 (via (at 65.479542 95.43934) (size 0.6) (drill 0.15) (layers "F.Cu" "B.Cu") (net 31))
 (segment (start 64.879542 97.312131) (end 64.879542 102.970068) (width 0.2) (layer "B.Cu") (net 31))
 (segment (start 65.197495 95.721387) (end 65.197495 96.994178) (width 0.2) (layer "B.Cu") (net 31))
 (segment (start 65.197495 96.994178) (end 64.879542 97.312131) (width 0.2) (layer "B.Cu") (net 31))
 (segment (start 65.479542 95.43934) (end 65.197495 95.721387) (width 0.2) (layer "B.Cu") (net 31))
 (segment (start 64.879542 102.970068) (end 63.92044 103.92917) (width 0.2) (layer "B.Cu") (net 31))
 (segment (start 71.56066 101.520458) (end 71.56066 103.88895) (width 0.2) (layer "F.Cu") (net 18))
 (segment (start 71.56066 103.88895) (end 71.52044 103.92917) (width 0.2) (layer "F.Cu") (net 18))
 (segment (start 59.970226 87.998831) (end 62.276422 87.998831) (width 0.2) (layer "F.Cu") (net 3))
 (segment (start 66.8584 93.742284) (end 67.176598 93.742284) (width 0.2) (layer "F.Cu") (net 3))
 (segment (start 58.936452 92.022702) (end 57.742182 92.022702) (width 0.2) (layer "F.Cu") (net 3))
 (segment (start 62.660645 89.544529) (end 66.8584 93.742284) (width 0.2) (layer "F.Cu") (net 3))
 (segment (start 57.651313 90.318913) (end 59.970226 88) (width 0.2) (layer "F.Cu") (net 3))
 (segment (start 62.660645 88.384223) (end 62.660645 89.544529) (width 0.2) (layer "F.Cu") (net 3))
 (segment (start 57.742182 92.022702) (end 57.651313 91.931833) (width 0.2) (layer "F.Cu") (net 3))
 (segment (start 62.276422 88) (end 62.660645 88.384223) (width 0.2) (layer "F.Cu") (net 3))
 (segment (start 57.651313 91.931833) (end 57.651313 90.318913) (width 0.2) (layer "F.Cu") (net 3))
 (segment (start 50.927151 103.923112) (end 52.083209 105.07917) (width 0.2) (layer "B.Cu") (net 3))
 (segment (start 51.479195 97.693112) (end 50.450805 97.693112) (width 0.2) (layer "B.Cu") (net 3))
 (segment (start 58.920151 89.050075) (end 58.920151 90.252156) (width 0.2) (layer "B.Cu") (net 3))
 (segment (start 49.777151 98.366766) (end 49.777151 102.773112) (width 0.2) (layer "B.Cu") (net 3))
 (segment (start 52.083209 105.07917) (end 57.69044 105.07917) (width 0.2) (layer "B.Cu") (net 3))
 (segment (start 57.69044 105.07917) (end 58.84044 103.92917) (width 0.2) (layer "B.Cu") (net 3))
 (segment (start 49.777151 102.773112) (end 50.927151 103.923112) (width 0.2) (layer "B.Cu") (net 3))
 (segment (start 50.450805 97.693112) (end 49.777151 98.366766) (width 0.2) (layer "B.Cu") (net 3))
 (segment (start 58.920151 90.252156) (end 51.479195 97.693112) (width 0.2) (layer "B.Cu") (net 3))
 (via (at 66.045227 94.873654) (size 0.6) (drill 0.15) (layers "F.Cu" "B.Cu") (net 30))
 (segment (start 65.762384 94.590811) (end 63.098799 94.590811) (width 0.2) (layer "B.Cu") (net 30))
 (segment (start 51.214382 101.383112) (end 50.927151 101.383112) (width 0.2) (layer "B.Cu") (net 30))
 (segment (start 66.045227 94.873654) (end 65.762384 94.590811) (width 0.2) (layer "B.Cu") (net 30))
 (segment (start 63.098799 94.590811) (end 53.76044 103.92917) (width 0.2) (layer "B.Cu") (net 30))
 (segment (start 53.76044 103.92917) (end 51.214382 101.383112) (width 0.2) (layer "B.Cu") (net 30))
 (segment (start 79.14044 103.92917) (end 78.226786 103.92917) (width 0.2) (layer "F.Cu") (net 21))
 (segment (start 78.226786 103.92917) (end 77.076786 102.77917) (width 0.2) (layer "F.Cu") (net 21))
 (segment (start 76.213484 102.77917) (end 73.257716 99.823402) (width 0.2) (layer "F.Cu") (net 21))
 (segment (start 77.076786 102.77917) (end 76.213484 102.77917) (width 0.2) (layer "F.Cu") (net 21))
 (via (at 66.045227 98.126346) (size 0.6) (drill 0.15) (layers "F.Cu" "B.Cu") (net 13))
 (segment (start 66.045227 100.993957) (end 68.98044 103.92917) (width 0.2) (layer "B.Cu") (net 13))
 (segment (start 66.045227 98.126346) (end 66.045227 100.993957) (width 0.2) (layer "B.Cu") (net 13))
 (segment (start 72.692031 100.389087) (end 76.232114 103.92917) (width 0.2) (layer "F.Cu") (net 20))
 (segment (start 76.232114 103.92917) (end 76.60044 103.92917) (width 0.2) (layer "F.Cu") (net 20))
 (via (at 65.479542 97.56066) (size 0.6) (drill 0.15) (layers "F.Cu" "B.Cu") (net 12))
 (segment (start 65.445227 102.913957) (end 66.46044 103.92917) (width 0.2) (layer "B.Cu") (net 12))
 (segment (start 65.445227 97.877817) (end 65.445227 102.913957) (width 0.2) (layer "B.Cu") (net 12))
 (segment (start 72.126346 100.954773) (end 74.06044 102.888867) (width 0.2) (layer "F.Cu") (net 19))
 (segment (start 74.06044 102.888867) (end 74.06044 103.92917) (width 0.2) (layer "F.Cu") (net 19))
 (segment (start 74.389087 98.692031) (end 74.67193 98.974874) (width 0.2) (layer "F.Cu") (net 11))
 (segment (start 75.66188 98.974874) (end 77.448248 97.188505) (width 0.2) (layer "F.Cu") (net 11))
 (segment (start 77.448248 97.188505) (end 77.448248 93.051752) (width 0.2) (layer "F.Cu") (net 11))
 (segment (start 77.448248 93.051752) (end 81.676543 88.823457) (width 0.2) (layer "F.Cu") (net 11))
 (segment (start 74.67193 98.974874) (end 75.66188 98.974874) (width 0.2) (layer "F.Cu") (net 11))
 (segment (start 76.248248 94.71155) (end 76.248248 91.00709) (width 0.2) (layer "F.Cu") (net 8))
 (segment (start 75.520458 95.43934) (end 76.248248 94.71155) (width 0.2) (layer "F.Cu") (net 8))
 (segment (start 76.248248 91.00709) (end 74.064615 88.823457) (width 0.2) (layer "F.Cu") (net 8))
 (via (at 61.509061 93.697016) (size 0.6) (drill 0.15) (layers "F.Cu" "B.Cu") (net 8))
 (segment (start 61.509061 93.697016) (end 64.706077 90.5) (width 0.2) (layer "B.Cu") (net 8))
 (segment (start 72.690226 90.5) (end 74.140151 89.050075) (width 0.2) (layer "B.Cu") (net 8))
 (segment (start 64.706077 90.5) (end 72.690226 90.5) (width 0.2) (layer "B.Cu") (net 8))
 (segment (start 69.43934 91.479542) (end 66.783255 88.823457) (width 0.2) (layer "F.Cu") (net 5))
 (segment (start 66.783255 88.823457) (end 66.464615 88.823457) (width 0.2) (layer "F.Cu") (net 5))
 (segment (start 68.308489 91.480062) (end 68.873654 92.045227) (width 0.2) (layer "F.Cu") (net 4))
 (segment (start 66.430138 91.480062) (end 68.308489 91.480062) (width 0.2) (layer "F.Cu") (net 4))
 (segment (start 64.000151 89.050075) (end 66.430138 91.480062) (width 0.2) (layer "F.Cu") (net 4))
 (segment (start 76.604615 88.823457) (end 76.5 88.928072) (width 0.2) (layer "F.Cu") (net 9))
 (segment (start 76.648248 88.86709) (end 76.604615 88.823457) (width 0.2) (layer "F.Cu") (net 9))
 (segment (start 76.648248 96.43287) (end 76.648248 88.86709) (width 0.2) (layer "F.Cu") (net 9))
 (segment (start 75.520458 97.56066) (end 76.648248 96.43287) (width 0.2) (layer "F.Cu") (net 9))
 (segment (start 75.131029 98.302602) (end 74.954773 98.126346) (width 0.2) (layer "F.Cu") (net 10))
 (segment (start 77.048248 97.02282) (end 75.768466 98.302602) (width 0.2) (layer "F.Cu") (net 10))
 (segment (start 75.768466 98.302602) (end 75.131029 98.302602) (width 0.2) (layer "F.Cu") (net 10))
 (segment (start 77.048248 90.919824) (end 77.048248 97.02282) (width 0.2) (layer "F.Cu") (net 10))
 (segment (start 79.144615 88.823457) (end 77.048248 90.919824) (width 0.2) (layer "F.Cu") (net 10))
 (segment (start 71.56066 91.479542) (end 68.984615 88.903497) (width 0.2) (layer "F.Cu") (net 6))
 (segment (start 72.302602 91.868971) (end 72.126346 92.045227) (width 0.2) (layer "F.Cu") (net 7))
 (segment (start 71.600151 89.050075) (end 72.302602 89.752526) (width 0.2) (layer "F.Cu") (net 7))
 (segment (start 72.302602 89.752526) (end 72.302602 91.868971) (width 0.2) (layer "F.Cu") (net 7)))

